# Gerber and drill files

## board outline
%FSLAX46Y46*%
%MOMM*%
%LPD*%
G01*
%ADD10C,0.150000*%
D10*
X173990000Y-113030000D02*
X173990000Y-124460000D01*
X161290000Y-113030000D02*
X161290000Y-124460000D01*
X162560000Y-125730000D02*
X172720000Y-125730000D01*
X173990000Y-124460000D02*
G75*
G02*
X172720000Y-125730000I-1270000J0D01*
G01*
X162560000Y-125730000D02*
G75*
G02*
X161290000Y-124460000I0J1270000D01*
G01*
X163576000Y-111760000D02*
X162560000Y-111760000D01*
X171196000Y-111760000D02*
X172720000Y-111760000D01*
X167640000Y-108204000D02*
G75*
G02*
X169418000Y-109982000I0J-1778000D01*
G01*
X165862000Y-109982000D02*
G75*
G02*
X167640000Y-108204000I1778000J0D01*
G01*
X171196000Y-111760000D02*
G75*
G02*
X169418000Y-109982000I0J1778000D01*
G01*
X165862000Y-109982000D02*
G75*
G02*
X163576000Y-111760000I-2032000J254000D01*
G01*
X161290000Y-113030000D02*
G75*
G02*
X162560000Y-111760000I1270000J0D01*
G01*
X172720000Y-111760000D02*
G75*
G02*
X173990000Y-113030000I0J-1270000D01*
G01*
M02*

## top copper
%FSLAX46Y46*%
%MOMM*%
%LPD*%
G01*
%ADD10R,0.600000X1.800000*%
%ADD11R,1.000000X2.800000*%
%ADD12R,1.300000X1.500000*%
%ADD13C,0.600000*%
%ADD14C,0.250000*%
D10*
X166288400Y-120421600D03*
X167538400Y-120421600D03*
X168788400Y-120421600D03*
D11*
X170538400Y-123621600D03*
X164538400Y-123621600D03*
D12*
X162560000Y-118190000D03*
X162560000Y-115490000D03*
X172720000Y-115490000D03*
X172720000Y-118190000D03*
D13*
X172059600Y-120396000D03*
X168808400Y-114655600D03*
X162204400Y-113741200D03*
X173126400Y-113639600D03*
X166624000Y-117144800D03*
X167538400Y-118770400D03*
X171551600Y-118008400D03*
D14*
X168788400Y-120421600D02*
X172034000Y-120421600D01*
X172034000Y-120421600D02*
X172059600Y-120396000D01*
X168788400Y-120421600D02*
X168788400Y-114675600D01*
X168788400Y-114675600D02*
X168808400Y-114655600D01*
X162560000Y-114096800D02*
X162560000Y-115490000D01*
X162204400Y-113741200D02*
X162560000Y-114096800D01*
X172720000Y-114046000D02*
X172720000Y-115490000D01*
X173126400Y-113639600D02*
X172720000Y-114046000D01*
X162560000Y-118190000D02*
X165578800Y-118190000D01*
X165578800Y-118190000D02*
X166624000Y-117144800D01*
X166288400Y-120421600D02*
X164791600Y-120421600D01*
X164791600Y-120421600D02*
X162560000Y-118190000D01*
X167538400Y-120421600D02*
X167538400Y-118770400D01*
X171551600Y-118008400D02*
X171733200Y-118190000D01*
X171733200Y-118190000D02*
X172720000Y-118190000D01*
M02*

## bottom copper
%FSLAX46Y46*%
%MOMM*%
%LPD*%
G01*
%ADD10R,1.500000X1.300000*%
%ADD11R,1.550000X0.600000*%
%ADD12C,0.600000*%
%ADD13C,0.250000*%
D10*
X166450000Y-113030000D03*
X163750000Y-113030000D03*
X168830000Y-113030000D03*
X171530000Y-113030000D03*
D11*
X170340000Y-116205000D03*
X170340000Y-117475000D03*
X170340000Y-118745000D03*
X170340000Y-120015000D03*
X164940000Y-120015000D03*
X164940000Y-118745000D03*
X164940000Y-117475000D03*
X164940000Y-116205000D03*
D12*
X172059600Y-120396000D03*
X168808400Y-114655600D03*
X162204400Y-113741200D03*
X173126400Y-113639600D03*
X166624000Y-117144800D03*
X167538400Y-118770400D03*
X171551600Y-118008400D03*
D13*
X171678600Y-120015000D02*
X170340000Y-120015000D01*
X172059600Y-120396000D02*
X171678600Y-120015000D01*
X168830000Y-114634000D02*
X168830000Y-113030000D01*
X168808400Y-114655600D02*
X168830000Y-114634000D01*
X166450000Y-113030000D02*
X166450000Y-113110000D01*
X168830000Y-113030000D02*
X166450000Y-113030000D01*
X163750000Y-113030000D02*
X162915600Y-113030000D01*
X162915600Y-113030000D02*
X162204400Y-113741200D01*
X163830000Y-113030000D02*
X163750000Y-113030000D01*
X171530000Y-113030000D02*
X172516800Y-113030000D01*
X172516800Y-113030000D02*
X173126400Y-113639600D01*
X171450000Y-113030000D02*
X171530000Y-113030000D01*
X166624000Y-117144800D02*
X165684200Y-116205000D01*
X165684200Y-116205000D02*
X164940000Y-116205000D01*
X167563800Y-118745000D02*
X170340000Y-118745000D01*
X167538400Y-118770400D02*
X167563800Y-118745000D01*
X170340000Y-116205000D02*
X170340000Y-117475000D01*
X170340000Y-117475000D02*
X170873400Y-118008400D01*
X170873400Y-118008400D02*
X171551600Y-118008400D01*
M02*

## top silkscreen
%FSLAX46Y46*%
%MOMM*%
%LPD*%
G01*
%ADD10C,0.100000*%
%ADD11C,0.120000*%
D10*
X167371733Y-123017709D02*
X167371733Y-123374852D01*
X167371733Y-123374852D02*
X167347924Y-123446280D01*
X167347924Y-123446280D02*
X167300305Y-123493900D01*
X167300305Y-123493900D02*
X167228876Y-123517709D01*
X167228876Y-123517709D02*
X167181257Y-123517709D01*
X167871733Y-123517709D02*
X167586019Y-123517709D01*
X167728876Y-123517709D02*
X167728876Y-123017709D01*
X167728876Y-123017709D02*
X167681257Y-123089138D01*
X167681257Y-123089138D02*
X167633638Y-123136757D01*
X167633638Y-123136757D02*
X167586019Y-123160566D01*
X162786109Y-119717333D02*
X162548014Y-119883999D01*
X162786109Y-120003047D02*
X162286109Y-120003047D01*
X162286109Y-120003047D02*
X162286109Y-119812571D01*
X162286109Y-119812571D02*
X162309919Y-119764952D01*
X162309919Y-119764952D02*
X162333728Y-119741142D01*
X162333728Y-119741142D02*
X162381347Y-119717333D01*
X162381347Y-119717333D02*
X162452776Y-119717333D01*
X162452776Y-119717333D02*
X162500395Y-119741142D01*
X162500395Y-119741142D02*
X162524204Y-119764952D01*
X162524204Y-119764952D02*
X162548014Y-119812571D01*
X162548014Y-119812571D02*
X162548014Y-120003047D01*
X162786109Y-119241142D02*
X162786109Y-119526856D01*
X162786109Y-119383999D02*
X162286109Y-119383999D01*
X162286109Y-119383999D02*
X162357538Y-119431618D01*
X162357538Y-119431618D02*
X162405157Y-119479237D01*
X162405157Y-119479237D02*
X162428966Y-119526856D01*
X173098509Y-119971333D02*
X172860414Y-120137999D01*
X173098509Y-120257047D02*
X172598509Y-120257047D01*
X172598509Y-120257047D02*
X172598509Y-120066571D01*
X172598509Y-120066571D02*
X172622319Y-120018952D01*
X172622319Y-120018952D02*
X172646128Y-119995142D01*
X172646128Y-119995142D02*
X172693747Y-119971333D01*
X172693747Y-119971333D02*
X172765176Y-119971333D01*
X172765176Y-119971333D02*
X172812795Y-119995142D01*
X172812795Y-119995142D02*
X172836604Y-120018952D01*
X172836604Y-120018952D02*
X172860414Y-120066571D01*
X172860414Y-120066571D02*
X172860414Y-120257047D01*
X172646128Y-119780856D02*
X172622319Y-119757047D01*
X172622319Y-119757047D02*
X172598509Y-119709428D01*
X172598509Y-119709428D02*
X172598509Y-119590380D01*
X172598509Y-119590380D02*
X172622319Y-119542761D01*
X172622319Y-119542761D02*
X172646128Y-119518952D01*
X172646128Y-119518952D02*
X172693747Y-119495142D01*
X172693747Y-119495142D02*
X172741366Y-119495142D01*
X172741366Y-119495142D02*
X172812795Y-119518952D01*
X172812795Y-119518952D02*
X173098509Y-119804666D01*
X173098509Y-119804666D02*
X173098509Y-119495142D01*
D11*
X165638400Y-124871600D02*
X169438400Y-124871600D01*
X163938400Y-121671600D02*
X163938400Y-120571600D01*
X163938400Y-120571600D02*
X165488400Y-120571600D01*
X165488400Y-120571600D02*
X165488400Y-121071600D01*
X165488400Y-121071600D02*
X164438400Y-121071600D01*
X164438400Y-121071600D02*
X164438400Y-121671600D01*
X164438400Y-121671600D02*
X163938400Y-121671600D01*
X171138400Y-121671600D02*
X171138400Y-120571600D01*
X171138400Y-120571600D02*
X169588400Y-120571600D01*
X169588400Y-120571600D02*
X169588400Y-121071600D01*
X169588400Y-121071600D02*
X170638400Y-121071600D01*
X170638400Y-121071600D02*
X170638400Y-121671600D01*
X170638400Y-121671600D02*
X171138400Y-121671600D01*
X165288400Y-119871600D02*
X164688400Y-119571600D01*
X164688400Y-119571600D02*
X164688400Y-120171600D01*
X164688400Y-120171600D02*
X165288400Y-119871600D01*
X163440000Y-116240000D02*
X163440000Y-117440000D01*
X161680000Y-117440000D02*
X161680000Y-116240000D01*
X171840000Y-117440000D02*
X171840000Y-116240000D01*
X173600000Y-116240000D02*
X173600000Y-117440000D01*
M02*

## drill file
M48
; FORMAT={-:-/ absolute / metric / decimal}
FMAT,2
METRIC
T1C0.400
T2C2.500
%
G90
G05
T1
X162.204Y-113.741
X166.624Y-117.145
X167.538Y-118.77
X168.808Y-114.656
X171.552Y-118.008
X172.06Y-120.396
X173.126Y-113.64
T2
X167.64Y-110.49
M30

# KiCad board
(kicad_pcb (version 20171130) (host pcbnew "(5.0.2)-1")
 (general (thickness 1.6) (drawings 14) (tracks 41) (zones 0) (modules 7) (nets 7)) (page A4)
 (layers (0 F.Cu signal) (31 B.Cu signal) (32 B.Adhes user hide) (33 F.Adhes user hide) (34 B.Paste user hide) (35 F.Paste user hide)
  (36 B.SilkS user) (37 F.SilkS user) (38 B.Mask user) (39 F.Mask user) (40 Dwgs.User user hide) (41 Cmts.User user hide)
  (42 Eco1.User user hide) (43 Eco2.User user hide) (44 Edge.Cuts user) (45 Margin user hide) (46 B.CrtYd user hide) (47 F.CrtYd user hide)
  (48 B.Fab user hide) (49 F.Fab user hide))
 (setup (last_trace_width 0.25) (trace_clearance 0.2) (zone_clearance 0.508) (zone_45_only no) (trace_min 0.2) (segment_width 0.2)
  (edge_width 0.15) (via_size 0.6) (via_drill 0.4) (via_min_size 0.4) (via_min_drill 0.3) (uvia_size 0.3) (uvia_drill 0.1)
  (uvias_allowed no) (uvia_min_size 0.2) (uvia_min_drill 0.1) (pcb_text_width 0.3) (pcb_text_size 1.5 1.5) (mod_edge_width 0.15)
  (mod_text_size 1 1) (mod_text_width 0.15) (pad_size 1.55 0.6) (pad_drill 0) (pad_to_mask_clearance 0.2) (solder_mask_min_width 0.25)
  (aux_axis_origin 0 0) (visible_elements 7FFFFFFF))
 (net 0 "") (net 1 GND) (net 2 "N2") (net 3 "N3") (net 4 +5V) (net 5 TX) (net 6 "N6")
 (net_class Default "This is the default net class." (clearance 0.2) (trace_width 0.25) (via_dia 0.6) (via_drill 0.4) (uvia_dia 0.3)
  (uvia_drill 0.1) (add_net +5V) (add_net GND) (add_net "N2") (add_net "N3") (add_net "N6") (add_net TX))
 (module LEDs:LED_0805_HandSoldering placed (layer B.Cu) (at 165.1 113.03 180)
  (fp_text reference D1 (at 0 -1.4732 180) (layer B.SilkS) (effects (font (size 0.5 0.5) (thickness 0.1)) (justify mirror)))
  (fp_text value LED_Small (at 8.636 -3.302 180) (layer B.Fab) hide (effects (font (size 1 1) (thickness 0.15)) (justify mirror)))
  (pad 1 smd rect (at -1.35 0 180) (size 1.5 1.3) (layers B.Cu B.Paste B.Mask) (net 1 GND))
  (pad 2 smd rect (at 1.35 0 180) (size 1.5 1.3) (layers B.Cu B.Paste B.Mask) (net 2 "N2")))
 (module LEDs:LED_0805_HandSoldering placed (layer B.Cu) (at 170.18 113.03)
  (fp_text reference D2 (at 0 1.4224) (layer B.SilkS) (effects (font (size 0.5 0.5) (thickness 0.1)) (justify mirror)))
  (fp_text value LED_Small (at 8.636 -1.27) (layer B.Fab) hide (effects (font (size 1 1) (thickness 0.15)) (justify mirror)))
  (pad 1 smd rect (at -1.35 0) (size 1.5 1.3) (layers B.Cu B.Paste B.Mask) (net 1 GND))
  (pad 2 smd rect (at 1.35 0) (size 1.5 1.3) (layers B.Cu B.Paste B.Mask) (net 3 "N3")))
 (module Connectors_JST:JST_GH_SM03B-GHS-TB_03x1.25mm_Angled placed (layer F.Cu) (at 167.5384 122.0216)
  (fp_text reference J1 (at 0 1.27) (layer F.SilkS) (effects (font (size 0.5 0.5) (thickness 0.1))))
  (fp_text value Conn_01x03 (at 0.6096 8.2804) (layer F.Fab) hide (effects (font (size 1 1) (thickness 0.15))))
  (fp_line (start -1.9 2.85) (end 1.9 2.85) (layer F.SilkS) (width 0.12))
  (fp_line (start -3.6 -0.35) (end -3.6 -1.45) (layer F.SilkS) (width 0.12))
  (fp_line (start -3.6 -1.45) (end -2.05 -1.45) (layer F.SilkS) (width 0.12))
  (fp_line (start -2.05 -1.45) (end -2.05 -0.95) (layer F.SilkS) (width 0.12))
  (fp_line (start -2.05 -0.95) (end -3.1 -0.95) (layer F.SilkS) (width 0.12))
  (fp_line (start -3.1 -0.95) (end -3.1 -0.35) (layer F.SilkS) (width 0.12))
  (fp_line (start -3.1 -0.35) (end -3.6 -0.35) (layer F.SilkS) (width 0.12))
  (fp_line (start 3.6 -0.35) (end 3.6 -1.45) (layer F.SilkS) (width 0.12))
  (fp_line (start 3.6 -1.45) (end 2.05 -1.45) (layer F.SilkS) (width 0.12))
  (fp_line (start 2.05 -1.45) (end 2.05 -0.95) (layer F.SilkS) (width 0.12))
  (fp_line (start 2.05 -0.95) (end 3.1 -0.95) (layer F.SilkS) (width 0.12))
  (fp_line (start 3.1 -0.95) (end 3.1 -0.35) (layer F.SilkS) (width 0.12))
  (fp_line (start 3.1 -0.35) (end 3.6 -0.35) (layer F.SilkS) (width 0.12))
  (fp_line (start -2.25 -2.15) (end -2.85 -2.45) (layer F.SilkS) (width 0.12))
  (fp_line (start -2.85 -2.45) (end -2.85 -1.85) (layer F.SilkS) (width 0.12))
  (fp_line (start -2.85 -1.85) (end -2.25 -2.15) (layer F.SilkS) (width 0.12))
  (pad 1 smd rect (at -1.25 -1.6) (size 0.6 1.8) (layers F.Cu F.Paste F.Mask) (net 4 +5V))
  (pad 2 smd rect (at 0 -1.6) (size 0.6 1.8) (layers F.Cu F.Paste F.Mask) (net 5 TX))
  (pad 3 smd rect (at 1.25 -1.6) (size 0.6 1.8) (layers F.Cu F.Paste F.Mask) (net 1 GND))
  (pad "" smd rect (at 3 1.6) (size 1 2.8) (layers F.Cu F.Paste F.Mask))
  (pad "" smd rect (at -3 1.6) (size 1 2.8) (layers F.Cu F.Paste F.Mask)))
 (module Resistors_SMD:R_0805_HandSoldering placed (layer F.Cu) (at 162.56 116.84 90)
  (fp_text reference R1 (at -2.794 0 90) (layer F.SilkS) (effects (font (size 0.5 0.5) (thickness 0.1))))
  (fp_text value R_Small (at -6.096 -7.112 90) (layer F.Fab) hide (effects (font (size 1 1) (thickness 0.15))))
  (fp_line (start 0.6 0.88) (end -0.6 0.88) (layer F.SilkS) (width 0.12))
  (fp_line (start -0.6 -0.88) (end 0.6 -0.88) (layer F.SilkS) (width 0.12))
  (pad 1 smd rect (at -1.35 0 90) (size 1.5 1.3) (layers F.Cu F.Paste F.Mask) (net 4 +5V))
  (pad 2 smd rect (at 1.35 0 90) (size 1.5 1.3) (layers F.Cu F.Paste F.Mask) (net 2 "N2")))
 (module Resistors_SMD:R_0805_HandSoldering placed (layer F.Cu) (at 172.72 116.84 270)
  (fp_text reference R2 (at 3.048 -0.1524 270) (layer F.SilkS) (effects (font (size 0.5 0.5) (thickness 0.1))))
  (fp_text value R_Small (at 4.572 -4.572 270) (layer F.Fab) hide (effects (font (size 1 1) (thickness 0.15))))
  (fp_line (start 0.6 0.88) (end -0.6 0.88) (layer F.SilkS) (width 0.12))
  (fp_line (start -0.6 -0.88) (end 0.6 -0.88) (layer F.SilkS) (width 0.12))
  (pad 1 smd rect (at -1.35 0 270) (size 1.5 1.3) (layers F.Cu F.Paste F.Mask) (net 3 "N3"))
  (pad 2 smd rect (at 1.35 0 270) (size 1.5 1.3) (layers F.Cu F.Paste F.Mask) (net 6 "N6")))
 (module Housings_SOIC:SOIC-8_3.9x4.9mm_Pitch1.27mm (layer B.Cu) (at 167.64 118.11 180)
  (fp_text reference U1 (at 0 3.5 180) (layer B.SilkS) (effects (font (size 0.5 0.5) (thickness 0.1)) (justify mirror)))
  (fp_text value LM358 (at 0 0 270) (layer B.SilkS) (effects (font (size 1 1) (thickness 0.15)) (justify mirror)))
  (pad 1 smd rect (at -2.7 1.905 180) (size 1.55 0.6) (layers B.Cu B.Paste B.Mask) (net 6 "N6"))
  (pad 2 smd rect (at -2.7 0.635 180) (size 1.55 0.6) (layers B.Cu B.Paste B.Mask) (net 6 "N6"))
  (pad 3 smd rect (at -2.7 -0.635 180) (size 1.55 0.6) (layers B.Cu B.Paste B.Mask) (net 5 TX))
  (pad 4 smd rect (at -2.7 -1.905 180) (size 1.55 0.6) (layers B.Cu B.Paste B.Mask) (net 1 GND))
  (pad 5 smd rect (at 2.7 -1.905 180) (size 1.55 0.6) (layers B.Cu B.Paste B.Mask))
  (pad 6 smd rect (at 2.7 -0.635 180) (size 1.55 0.6) (layers B.Cu B.Paste B.Mask))
  (pad 7 smd rect (at 2.7 0.635 180) (size 1.55 0.6) (layers B.Cu B.Paste B.Mask))
  (pad 8 smd rect (at 2.7 1.905 180) (size 1.55 0.6) (layers B.Cu B.Paste B.Mask) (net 4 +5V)))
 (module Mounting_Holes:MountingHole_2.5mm (layer F.Cu) (at 167.64 110.49)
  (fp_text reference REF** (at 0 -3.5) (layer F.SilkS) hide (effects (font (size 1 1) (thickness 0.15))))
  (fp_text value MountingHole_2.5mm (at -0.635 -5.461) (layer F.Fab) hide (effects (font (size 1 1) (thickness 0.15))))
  (pad 1 np_thru_hole circle (at 0 0) (size 2.5 2.5) (drill 2.5) (layers *.Cu *.Mask)))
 (gr_line (start 173.99 113.03) (end 173.99 124.46) (angle 90) (layer Edge.Cuts) (width 0.15))
 (gr_line (start 161.29 113.03) (end 161.29 124.46) (angle 90) (layer Edge.Cuts) (width 0.15))
 (gr_line (start 162.56 125.73) (end 172.72 125.73) (angle 90) (layer Edge.Cuts) (width 0.15))
 (gr_arc (start 172.72 124.46) (end 173.99 124.46) (angle 90) (layer Edge.Cuts) (width 0.15))
 (gr_arc (start 162.56 124.46) (end 162.56 125.73) (angle 90) (layer Edge.Cuts) (width 0.15))
 (gr_line (start 163.576 111.76) (end 162.56 111.76) (angle 90) (layer Edge.Cuts) (width 0.15))
 (gr_line (start 171.196 111.76) (end 172.72 111.76) (angle 90) (layer Edge.Cuts) (width 0.15))
 (gr_arc (start 167.64 109.982) (end 167.64 108.204) (angle 90) (layer Edge.Cuts) (width 0.15))
 (gr_arc (start 167.64 109.982) (end 165.862 109.982) (angle 90) (layer Edge.Cuts) (width 0.15))
 (gr_arc (start 171.196 109.982) (end 171.196 111.76) (angle 90) (layer Edge.Cuts) (width 0.15))
 (gr_arc (start 163.83 109.728) (end 165.862 109.982) (angle 90) (layer Edge.Cuts) (width 0.15))
 (gr_arc (start 162.56 113.03) (end 161.29 113.03) (angle 90) (layer Edge.Cuts) (width 0.15))
 (gr_arc (start 172.72 113.03) (end 172.72 111.76) (angle 90) (layer Edge.Cuts) (width 0.15))
 (segment (start 168.7884 120.4216) (end 172.034 120.4216) (width 0.25) (layer F.Cu) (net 1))
 (segment (start 171.6786 120.015) (end 170.34 120.015) (width 0.25) (layer B.Cu) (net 1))
 (segment (start 172.0596 120.396) (end 171.6786 120.015) (width 0.25) (layer B.Cu) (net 1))
 (via (at 172.0596 120.396) (size 0.6) (drill 0.4) (layers F.Cu B.Cu) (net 1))
 (segment (start 172.034 120.4216) (end 172.0596 120.396) (width 0.25) (layer F.Cu) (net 1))
 (segment (start 168.7884 120.4216) (end 168.7884 114.6756) (width 0.25) (layer F.Cu) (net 1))
 (segment (start 168.83 114.634) (end 168.83 113.03) (width 0.25) (layer B.Cu) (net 1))
 (segment (start 168.8084 114.6556) (end 168.83 114.634) (width 0.25) (layer B.Cu) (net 1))
 (via (at 168.8084 114.6556) (size 0.6) (drill 0.4) (layers F.Cu B.Cu) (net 1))
 (segment (start 168.7884 114.6756) (end 168.8084 114.6556) (width 0.25) (layer F.Cu) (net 1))
 (segment (start 166.45 113.03) (end 166.45 113.11) (width 0.25) (layer B.Cu) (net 1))
 (segment (start 168.83 113.03) (end 166.45 113.03) (width 0.25) (layer B.Cu) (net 1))
 (segment (start 163.75 113.03) (end 162.9156 113.03) (width 0.25) (layer B.Cu) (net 2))
 (segment (start 162.56 114.0968) (end 162.56 115.49) (width 0.25) (layer F.Cu) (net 2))
 (segment (start 162.2044 113.7412) (end 162.56 114.0968) (width 0.25) (layer F.Cu) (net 2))
 (via (at 162.2044 113.7412) (size 0.6) (drill 0.4) (layers F.Cu B.Cu) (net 2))
 (segment (start 162.9156 113.03) (end 162.2044 113.7412) (width 0.25) (layer B.Cu) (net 2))
 (segment (start 163.83 113.03) (end 163.75 113.03) (width 0.25) (layer B.Cu) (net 2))
 (segment (start 171.53 113.03) (end 172.5168 113.03) (width 0.25) (layer B.Cu) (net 3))
 (segment (start 172.72 114.046) (end 172.72 115.49) (width 0.25) (layer F.Cu) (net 3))
 (segment (start 173.1264 113.6396) (end 172.72 114.046) (width 0.25) (layer F.Cu) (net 3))
 (via (at 173.1264 113.6396) (size 0.6) (drill 0.4) (layers F.Cu B.Cu) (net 3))
 (segment (start 172.5168 113.03) (end 173.1264 113.6396) (width 0.25) (layer B.Cu) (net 3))
 (segment (start 171.45 113.03) (end 171.53 113.03) (width 0.25) (layer B.Cu) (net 3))
 (segment (start 162.56 118.19) (end 165.5788 118.19) (width 0.25) (layer F.Cu) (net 4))
 (segment (start 166.624 117.1448) (end 165.6842 116.205) (width 0.25) (layer B.Cu) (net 4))
 (via (at 166.624 117.1448) (size 0.6) (drill 0.4) (layers F.Cu B.Cu) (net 4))
 (segment (start 165.5788 118.19) (end 166.624 117.1448) (width 0.25) (layer F.Cu) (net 4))
 (segment (start 165.6842 116.205) (end 164.94 116.205) (width 0.25) (layer B.Cu) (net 4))
 (segment (start 166.2884 120.4216) (end 164.7916 120.4216) (width 0.25) (layer F.Cu) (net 4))
 (segment (start 164.7916 120.4216) (end 162.56 118.19) (width 0.25) (layer F.Cu) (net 4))
 (segment (start 167.5384 120.4216) (end 167.5384 118.7704) (width 0.25) (layer F.Cu) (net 5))
 (segment (start 167.5638 118.745) (end 170.34 118.745) (width 0.25) (layer B.Cu) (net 5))
 (segment (start 167.5384 118.7704) (end 167.5638 118.745) (width 0.25) (layer B.Cu) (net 5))
 (via (at 167.5384 118.7704) (size 0.6) (drill 0.4) (layers F.Cu B.Cu) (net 5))
 (segment (start 170.34 116.205) (end 170.34 117.475) (width 0.25) (layer B.Cu) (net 6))
 (segment (start 170.34 117.475) (end 170.8734 118.0084) (width 0.25) (layer B.Cu) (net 6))
 (segment (start 170.8734 118.0084) (end 171.5516 118.0084) (width 0.25) (layer B.Cu) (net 6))
 (via (at 171.5516 118.0084) (size 0.6) (drill 0.4) (layers F.Cu B.Cu) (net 6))
 (segment (start 171.5516 118.0084) (end 171.7332 118.19) (width 0.25) (layer F.Cu) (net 6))
 (segment (start 171.7332 118.19) (end 172.72 118.19) (width 0.25) (layer F.Cu) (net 6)))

